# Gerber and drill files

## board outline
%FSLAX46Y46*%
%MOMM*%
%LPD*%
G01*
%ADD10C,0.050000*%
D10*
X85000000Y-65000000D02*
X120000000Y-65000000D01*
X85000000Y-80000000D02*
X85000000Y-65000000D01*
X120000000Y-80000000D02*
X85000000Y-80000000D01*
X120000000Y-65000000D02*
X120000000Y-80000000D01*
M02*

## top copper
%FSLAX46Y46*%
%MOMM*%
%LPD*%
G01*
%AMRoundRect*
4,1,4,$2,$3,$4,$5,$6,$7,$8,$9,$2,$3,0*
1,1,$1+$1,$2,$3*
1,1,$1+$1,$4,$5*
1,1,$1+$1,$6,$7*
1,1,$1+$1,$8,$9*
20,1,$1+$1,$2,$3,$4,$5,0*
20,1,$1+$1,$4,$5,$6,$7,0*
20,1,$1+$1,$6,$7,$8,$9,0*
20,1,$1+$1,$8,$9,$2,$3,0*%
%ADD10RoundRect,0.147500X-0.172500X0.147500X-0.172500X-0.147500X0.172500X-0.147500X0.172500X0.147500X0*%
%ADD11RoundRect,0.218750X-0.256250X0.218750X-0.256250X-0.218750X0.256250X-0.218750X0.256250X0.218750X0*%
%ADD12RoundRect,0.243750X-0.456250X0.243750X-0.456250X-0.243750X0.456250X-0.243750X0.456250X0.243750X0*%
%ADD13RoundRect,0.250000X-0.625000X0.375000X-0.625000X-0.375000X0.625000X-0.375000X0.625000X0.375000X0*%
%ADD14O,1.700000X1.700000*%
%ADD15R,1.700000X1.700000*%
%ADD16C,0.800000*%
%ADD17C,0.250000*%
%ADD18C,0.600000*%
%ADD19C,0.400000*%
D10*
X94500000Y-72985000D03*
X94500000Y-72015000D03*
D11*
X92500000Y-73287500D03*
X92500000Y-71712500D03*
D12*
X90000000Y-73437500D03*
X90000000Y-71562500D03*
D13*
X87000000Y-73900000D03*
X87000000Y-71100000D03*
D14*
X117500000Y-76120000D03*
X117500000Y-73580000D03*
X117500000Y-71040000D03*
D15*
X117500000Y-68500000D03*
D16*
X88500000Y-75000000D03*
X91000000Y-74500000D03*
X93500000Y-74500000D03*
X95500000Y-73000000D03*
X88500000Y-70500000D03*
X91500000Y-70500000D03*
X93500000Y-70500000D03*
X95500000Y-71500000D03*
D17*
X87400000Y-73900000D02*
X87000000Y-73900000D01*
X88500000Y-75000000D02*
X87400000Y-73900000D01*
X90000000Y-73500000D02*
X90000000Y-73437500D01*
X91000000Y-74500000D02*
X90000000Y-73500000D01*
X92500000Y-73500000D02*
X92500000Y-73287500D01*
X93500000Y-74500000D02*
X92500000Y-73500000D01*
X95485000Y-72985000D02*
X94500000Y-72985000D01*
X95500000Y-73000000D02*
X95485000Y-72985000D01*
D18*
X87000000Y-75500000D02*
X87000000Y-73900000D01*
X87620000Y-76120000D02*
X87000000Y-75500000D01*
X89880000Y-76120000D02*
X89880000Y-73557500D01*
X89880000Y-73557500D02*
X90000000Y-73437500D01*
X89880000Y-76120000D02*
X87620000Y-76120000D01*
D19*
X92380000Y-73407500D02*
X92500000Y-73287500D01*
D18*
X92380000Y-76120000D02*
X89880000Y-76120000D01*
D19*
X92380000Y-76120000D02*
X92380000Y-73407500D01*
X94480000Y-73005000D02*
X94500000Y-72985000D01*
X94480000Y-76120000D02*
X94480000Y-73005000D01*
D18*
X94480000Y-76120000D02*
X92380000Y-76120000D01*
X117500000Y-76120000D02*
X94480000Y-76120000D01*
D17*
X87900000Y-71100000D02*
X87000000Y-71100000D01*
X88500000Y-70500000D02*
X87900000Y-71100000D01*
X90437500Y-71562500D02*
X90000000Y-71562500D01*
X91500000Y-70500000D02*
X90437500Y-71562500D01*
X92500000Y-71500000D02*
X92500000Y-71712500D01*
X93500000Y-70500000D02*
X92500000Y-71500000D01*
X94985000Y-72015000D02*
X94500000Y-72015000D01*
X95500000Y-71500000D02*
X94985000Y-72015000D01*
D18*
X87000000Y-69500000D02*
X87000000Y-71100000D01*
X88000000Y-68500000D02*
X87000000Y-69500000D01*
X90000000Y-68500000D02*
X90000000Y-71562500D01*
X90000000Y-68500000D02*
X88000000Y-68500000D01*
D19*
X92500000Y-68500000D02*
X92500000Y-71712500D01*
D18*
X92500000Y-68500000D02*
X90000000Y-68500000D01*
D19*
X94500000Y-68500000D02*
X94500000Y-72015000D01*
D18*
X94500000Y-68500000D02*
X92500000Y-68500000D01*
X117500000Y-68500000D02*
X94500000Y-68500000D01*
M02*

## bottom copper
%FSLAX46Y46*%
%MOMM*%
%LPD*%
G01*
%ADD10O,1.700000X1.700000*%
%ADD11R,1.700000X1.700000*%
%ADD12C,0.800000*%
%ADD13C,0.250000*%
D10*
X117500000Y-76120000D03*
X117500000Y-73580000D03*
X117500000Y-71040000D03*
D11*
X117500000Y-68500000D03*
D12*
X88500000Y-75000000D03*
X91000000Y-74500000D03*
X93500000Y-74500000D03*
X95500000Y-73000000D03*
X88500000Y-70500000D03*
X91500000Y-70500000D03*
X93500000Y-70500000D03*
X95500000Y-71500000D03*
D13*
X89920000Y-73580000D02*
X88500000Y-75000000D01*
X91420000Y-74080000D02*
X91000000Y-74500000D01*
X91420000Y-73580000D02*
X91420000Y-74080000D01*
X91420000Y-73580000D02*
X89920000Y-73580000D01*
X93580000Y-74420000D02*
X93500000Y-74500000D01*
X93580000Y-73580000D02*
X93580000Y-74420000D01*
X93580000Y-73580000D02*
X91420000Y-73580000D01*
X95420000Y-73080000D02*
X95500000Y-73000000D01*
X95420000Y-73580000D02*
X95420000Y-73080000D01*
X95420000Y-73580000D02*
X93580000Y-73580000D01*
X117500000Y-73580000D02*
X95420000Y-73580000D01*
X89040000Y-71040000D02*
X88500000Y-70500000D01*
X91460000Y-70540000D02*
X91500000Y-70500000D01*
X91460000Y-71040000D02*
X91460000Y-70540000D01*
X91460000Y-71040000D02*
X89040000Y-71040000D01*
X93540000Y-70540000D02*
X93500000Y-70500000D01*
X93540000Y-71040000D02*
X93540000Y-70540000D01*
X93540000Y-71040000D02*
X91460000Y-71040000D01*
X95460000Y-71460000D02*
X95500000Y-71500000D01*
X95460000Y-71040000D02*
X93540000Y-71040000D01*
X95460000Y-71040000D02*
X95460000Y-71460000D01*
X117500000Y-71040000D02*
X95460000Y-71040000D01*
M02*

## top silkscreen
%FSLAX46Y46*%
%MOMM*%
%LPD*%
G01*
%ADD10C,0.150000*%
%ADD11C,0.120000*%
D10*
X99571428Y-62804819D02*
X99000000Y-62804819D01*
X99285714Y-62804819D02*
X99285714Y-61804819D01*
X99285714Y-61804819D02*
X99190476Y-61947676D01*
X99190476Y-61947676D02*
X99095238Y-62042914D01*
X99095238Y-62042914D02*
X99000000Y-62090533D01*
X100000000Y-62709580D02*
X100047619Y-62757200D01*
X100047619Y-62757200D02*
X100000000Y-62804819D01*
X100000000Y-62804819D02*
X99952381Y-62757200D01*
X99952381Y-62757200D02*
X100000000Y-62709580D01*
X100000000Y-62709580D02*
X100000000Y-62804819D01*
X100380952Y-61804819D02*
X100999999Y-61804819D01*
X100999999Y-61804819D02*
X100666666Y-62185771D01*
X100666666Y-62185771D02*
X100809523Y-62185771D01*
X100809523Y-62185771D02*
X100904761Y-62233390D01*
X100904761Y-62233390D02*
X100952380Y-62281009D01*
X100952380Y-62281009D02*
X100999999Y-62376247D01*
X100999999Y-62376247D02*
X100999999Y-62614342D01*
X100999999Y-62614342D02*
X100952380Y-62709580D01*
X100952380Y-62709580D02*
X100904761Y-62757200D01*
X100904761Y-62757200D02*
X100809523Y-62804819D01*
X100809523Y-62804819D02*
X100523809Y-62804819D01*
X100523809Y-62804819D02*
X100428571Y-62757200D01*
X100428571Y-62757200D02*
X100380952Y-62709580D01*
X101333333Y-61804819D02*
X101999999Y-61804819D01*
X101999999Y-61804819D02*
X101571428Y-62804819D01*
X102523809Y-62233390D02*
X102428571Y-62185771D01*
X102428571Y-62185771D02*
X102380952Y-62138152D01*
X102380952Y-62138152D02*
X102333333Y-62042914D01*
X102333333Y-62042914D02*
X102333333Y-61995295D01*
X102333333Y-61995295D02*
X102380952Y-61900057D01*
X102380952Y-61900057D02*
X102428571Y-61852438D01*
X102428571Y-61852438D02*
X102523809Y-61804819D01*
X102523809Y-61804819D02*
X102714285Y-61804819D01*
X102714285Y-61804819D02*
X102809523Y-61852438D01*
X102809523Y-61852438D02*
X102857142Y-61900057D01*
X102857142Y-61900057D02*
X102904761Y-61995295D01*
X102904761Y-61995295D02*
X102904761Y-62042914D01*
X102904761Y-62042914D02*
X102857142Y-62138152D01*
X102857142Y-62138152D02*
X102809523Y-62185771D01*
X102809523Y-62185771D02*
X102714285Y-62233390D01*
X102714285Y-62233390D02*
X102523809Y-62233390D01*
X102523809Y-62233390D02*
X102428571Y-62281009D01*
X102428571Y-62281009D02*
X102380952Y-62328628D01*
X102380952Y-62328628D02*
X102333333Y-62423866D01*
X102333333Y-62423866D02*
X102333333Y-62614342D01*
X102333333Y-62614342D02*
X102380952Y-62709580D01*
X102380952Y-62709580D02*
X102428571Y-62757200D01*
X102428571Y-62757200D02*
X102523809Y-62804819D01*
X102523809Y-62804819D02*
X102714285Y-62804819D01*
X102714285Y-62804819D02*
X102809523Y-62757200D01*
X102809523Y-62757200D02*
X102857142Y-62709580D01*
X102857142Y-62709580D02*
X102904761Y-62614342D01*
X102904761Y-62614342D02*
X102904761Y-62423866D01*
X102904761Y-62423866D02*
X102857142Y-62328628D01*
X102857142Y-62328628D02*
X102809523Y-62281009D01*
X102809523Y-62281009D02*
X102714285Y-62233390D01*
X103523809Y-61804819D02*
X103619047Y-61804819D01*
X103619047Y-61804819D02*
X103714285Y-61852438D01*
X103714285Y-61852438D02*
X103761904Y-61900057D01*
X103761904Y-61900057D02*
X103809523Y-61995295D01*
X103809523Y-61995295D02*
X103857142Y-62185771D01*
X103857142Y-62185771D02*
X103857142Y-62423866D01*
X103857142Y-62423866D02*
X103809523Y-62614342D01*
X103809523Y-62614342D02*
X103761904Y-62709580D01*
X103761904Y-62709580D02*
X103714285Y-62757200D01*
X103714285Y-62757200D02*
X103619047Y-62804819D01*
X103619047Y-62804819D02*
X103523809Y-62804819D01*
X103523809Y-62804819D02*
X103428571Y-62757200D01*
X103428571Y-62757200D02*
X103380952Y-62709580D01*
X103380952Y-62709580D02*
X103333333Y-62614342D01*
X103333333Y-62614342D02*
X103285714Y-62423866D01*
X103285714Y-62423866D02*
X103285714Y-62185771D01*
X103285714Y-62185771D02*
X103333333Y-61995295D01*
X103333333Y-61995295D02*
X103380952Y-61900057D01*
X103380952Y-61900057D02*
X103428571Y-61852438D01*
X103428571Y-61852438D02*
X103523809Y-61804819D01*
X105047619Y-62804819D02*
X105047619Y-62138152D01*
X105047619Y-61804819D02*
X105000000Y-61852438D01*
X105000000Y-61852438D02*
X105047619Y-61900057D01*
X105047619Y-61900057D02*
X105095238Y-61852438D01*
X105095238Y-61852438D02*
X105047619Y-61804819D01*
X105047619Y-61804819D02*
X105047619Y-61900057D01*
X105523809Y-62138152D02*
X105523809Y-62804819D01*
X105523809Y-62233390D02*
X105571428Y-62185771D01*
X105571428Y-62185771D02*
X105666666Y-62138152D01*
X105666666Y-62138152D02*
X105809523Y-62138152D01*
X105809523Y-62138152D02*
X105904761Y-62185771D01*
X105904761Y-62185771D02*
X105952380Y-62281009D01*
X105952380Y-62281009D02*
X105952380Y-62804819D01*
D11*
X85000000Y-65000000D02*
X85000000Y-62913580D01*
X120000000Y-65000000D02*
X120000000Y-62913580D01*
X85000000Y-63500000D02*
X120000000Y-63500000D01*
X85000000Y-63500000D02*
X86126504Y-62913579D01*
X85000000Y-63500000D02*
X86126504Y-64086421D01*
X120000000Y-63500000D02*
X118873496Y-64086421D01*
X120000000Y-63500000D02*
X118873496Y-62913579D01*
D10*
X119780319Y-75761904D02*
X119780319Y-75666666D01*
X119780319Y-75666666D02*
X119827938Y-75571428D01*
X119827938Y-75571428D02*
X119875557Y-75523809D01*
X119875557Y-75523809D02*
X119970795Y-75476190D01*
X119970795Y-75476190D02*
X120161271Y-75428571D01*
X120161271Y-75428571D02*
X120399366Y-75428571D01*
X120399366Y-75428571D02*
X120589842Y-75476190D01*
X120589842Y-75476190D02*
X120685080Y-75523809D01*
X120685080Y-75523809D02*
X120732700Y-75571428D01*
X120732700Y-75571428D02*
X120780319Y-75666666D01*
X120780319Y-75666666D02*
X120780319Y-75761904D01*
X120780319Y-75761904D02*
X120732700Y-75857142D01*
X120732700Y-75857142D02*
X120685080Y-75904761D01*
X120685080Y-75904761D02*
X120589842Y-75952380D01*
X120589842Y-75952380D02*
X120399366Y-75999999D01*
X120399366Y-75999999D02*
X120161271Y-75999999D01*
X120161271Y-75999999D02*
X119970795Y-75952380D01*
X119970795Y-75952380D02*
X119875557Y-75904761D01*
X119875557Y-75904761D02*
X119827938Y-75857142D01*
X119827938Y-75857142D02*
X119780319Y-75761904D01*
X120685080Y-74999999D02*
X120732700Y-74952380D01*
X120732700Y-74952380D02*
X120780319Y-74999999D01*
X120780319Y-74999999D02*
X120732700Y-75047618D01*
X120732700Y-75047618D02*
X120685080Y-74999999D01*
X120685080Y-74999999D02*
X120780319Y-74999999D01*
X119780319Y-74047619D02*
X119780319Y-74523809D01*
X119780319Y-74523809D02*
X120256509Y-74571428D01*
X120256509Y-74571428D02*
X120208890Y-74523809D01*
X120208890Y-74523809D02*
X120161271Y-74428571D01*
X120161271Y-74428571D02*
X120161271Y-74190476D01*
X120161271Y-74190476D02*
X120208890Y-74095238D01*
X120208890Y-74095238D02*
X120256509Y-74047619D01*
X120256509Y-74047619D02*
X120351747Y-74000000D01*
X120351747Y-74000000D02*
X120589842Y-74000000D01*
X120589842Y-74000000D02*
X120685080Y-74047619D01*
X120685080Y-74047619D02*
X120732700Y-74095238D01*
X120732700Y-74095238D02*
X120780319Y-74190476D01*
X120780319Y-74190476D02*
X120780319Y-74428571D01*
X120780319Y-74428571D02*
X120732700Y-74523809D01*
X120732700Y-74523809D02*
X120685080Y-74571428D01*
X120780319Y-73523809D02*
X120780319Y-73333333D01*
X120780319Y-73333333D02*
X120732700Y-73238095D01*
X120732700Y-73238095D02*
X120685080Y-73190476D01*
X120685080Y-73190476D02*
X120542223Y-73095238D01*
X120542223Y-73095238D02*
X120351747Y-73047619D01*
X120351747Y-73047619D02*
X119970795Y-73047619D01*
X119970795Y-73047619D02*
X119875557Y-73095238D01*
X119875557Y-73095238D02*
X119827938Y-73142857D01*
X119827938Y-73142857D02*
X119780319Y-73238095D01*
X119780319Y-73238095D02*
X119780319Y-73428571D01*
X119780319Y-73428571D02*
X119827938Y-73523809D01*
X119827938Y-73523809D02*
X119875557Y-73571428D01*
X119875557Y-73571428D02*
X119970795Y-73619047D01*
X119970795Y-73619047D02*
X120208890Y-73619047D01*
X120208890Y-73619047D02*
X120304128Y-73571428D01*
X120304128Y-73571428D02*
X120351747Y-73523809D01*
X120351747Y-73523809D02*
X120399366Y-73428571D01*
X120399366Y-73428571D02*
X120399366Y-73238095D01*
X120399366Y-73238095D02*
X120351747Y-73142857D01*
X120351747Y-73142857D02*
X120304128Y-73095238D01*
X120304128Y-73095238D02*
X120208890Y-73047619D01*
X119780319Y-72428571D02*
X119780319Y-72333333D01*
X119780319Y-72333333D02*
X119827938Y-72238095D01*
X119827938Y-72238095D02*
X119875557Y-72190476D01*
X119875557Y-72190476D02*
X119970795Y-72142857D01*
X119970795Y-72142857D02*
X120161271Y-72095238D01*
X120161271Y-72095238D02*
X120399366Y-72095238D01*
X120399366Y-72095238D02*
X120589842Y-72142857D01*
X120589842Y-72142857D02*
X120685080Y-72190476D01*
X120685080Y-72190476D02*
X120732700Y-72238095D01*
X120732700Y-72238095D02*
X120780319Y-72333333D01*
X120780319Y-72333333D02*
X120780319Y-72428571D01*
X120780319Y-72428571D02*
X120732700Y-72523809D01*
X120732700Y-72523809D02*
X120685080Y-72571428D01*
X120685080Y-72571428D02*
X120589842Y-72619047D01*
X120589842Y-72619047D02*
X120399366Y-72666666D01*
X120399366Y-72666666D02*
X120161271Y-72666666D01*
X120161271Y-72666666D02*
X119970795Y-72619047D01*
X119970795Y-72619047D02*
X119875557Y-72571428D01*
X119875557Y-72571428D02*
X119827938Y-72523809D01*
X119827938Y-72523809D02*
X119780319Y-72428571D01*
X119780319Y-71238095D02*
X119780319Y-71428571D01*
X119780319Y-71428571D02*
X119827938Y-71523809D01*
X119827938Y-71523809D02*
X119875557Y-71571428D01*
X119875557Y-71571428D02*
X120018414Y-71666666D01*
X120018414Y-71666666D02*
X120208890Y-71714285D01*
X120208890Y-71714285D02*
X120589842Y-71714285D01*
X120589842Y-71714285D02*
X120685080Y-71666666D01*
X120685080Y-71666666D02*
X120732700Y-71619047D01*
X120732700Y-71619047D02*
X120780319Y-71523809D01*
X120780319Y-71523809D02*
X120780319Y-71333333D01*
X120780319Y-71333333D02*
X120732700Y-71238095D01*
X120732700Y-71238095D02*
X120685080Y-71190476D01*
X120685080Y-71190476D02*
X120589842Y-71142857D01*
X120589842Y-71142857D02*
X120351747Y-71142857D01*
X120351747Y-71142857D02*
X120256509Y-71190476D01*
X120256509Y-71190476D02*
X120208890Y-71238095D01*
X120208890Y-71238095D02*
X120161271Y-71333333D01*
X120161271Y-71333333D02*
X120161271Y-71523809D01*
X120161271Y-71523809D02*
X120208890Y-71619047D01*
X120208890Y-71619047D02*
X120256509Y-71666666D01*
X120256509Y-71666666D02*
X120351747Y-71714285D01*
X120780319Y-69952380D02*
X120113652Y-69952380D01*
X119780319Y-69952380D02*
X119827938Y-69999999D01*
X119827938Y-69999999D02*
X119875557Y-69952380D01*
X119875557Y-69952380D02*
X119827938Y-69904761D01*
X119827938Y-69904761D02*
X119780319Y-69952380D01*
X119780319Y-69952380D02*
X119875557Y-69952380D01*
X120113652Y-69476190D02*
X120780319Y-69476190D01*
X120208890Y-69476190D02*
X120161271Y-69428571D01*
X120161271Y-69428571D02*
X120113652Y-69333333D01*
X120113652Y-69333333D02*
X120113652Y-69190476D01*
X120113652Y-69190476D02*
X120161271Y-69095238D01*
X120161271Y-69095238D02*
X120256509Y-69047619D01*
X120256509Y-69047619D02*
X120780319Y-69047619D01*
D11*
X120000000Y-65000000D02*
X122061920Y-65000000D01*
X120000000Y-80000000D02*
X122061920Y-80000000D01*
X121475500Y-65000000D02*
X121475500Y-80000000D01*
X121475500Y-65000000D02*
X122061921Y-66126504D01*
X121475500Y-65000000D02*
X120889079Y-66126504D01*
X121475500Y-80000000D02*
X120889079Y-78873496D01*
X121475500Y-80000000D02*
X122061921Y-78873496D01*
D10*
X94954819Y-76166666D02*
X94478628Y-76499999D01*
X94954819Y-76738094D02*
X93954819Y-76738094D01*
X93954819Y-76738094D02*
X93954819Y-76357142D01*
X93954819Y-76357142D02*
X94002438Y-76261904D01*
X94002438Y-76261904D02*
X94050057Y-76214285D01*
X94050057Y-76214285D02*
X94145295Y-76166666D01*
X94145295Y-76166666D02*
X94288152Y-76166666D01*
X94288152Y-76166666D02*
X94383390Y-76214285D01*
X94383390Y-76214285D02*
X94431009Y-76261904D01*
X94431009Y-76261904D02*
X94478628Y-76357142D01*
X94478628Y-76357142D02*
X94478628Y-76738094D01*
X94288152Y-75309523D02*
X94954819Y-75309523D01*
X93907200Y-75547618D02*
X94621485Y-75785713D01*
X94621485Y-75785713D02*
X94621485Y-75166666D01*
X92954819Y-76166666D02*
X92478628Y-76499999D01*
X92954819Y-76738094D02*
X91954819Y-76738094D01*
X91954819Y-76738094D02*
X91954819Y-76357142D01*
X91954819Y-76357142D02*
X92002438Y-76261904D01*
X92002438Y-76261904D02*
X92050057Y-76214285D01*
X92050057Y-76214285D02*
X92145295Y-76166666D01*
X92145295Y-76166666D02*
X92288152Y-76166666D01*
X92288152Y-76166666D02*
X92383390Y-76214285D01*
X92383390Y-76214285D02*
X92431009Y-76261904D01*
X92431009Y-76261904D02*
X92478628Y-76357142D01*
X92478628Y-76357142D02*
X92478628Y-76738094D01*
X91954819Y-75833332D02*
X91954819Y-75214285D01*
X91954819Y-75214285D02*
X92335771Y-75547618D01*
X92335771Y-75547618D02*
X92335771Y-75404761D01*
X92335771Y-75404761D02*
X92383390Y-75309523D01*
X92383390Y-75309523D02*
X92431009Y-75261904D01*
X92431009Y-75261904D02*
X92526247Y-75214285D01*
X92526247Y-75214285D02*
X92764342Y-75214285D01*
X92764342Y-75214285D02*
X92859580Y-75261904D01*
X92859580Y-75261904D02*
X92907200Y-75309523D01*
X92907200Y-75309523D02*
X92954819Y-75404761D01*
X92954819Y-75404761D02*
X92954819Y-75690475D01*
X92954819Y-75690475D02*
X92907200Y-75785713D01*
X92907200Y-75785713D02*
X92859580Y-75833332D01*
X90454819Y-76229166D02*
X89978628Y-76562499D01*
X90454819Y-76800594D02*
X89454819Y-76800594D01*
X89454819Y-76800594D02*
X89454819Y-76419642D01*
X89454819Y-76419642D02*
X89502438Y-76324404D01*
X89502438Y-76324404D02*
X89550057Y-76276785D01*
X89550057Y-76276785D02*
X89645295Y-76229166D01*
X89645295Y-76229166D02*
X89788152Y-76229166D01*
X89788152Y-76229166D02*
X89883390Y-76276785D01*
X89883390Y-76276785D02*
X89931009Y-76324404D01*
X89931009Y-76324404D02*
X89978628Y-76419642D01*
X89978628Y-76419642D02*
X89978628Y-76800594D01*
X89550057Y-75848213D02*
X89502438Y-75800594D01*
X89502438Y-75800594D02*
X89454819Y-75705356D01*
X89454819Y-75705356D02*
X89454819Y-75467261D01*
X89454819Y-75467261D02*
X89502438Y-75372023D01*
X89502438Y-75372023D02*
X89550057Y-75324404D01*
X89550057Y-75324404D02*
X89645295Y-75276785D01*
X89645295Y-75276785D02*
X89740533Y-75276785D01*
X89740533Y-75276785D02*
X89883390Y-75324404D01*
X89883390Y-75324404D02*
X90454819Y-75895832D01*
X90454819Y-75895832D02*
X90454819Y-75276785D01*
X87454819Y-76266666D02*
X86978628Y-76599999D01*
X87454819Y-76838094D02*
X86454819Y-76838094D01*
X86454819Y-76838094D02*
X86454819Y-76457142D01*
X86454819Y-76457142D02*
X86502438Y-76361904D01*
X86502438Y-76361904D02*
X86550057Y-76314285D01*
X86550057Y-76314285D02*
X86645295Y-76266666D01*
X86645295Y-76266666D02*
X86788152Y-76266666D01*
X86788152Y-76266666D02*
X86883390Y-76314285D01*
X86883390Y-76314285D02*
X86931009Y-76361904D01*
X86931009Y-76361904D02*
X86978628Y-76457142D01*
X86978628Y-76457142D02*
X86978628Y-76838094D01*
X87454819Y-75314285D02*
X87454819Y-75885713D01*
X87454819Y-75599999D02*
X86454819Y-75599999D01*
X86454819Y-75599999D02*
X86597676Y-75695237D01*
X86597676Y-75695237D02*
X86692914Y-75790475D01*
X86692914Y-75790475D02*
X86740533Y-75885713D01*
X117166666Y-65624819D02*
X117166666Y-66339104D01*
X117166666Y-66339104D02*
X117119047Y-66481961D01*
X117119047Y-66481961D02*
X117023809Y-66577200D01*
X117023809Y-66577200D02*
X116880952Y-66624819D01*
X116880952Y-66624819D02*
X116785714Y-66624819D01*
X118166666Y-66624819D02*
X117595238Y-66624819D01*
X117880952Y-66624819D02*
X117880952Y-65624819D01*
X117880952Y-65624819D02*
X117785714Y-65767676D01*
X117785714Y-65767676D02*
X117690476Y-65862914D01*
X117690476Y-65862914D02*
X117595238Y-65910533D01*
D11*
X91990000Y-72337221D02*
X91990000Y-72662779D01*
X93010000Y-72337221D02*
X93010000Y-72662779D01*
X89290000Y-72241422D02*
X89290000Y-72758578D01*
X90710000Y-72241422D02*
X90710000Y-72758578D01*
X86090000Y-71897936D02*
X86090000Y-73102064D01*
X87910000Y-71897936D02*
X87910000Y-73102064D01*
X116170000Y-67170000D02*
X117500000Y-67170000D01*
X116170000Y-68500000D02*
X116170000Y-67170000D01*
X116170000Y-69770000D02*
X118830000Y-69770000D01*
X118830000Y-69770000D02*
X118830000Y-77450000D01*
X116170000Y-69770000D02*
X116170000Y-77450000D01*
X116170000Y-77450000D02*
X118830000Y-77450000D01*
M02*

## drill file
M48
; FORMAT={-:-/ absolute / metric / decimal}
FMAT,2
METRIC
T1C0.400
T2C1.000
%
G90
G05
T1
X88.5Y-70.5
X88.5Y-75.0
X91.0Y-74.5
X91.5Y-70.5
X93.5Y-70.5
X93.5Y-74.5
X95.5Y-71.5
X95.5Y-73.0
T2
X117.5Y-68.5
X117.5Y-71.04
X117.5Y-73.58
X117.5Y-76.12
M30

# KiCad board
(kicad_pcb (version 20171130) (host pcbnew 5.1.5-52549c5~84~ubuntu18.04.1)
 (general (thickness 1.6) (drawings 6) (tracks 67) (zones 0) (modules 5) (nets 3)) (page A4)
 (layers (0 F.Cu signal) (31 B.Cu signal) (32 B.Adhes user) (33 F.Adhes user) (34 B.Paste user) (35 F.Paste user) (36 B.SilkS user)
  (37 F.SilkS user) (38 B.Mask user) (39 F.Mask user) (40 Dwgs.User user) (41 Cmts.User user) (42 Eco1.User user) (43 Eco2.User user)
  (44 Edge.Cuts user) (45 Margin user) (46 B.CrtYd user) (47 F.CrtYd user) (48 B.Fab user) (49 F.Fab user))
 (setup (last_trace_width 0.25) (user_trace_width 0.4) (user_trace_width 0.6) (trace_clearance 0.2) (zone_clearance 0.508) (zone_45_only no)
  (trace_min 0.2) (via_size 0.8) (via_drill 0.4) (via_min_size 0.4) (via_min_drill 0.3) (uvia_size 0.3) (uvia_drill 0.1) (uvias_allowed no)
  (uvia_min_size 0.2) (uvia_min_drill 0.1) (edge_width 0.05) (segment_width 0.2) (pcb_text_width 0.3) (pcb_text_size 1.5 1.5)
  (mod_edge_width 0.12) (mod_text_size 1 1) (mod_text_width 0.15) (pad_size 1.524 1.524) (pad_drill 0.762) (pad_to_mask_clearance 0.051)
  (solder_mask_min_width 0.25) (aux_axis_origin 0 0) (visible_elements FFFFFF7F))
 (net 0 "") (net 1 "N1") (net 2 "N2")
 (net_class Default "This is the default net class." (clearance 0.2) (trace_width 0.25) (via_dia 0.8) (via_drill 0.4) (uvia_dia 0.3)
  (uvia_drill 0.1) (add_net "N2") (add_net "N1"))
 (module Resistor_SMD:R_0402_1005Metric (layer F.Cu) (at 94.5 72.5 270)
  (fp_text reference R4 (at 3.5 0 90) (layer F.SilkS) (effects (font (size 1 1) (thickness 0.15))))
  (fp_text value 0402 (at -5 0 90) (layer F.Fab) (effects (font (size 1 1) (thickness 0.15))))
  (pad 2 smd roundrect (at 0.485 0 270) (size 0.59 0.64) (layers F.Cu F.Paste F.Mask) (roundrect_rratio 0.25) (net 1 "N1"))
  (pad 1 smd roundrect (at -0.485 0 270) (size 0.59 0.64) (layers F.Cu F.Paste F.Mask) (roundrect_rratio 0.25) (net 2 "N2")))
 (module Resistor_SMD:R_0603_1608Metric (layer F.Cu) (at 92.5 72.5 270)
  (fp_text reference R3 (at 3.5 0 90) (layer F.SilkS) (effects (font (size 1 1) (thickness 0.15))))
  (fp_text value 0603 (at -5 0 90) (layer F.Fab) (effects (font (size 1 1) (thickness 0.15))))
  (fp_line (start -0.162779 0.51) (end 0.162779 0.51) (layer F.SilkS) (width 0.12))
  (fp_line (start -0.162779 -0.51) (end 0.162779 -0.51) (layer F.SilkS) (width 0.12))
  (pad 2 smd roundrect (at 0.7875 0 270) (size 0.875 0.95) (layers F.Cu F.Paste F.Mask) (roundrect_rratio 0.25) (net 1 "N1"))
  (pad 1 smd roundrect (at -0.7875 0 270) (size 0.875 0.95) (layers F.Cu F.Paste F.Mask) (roundrect_rratio 0.25) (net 2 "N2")))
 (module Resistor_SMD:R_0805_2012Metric (layer F.Cu) (at 90 72.5 270)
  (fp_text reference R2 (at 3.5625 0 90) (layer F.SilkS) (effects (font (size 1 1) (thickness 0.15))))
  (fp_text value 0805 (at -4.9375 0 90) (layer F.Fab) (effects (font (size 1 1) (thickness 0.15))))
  (fp_line (start -0.258578 0.71) (end 0.258578 0.71) (layer F.SilkS) (width 0.12))
  (fp_line (start -0.258578 -0.71) (end 0.258578 -0.71) (layer F.SilkS) (width 0.12))
  (pad 2 smd roundrect (at 0.9375 0 270) (size 0.975 1.4) (layers F.Cu F.Paste F.Mask) (roundrect_rratio 0.25) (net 1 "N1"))
  (pad 1 smd roundrect (at -0.9375 0 270) (size 0.975 1.4) (layers F.Cu F.Paste F.Mask) (roundrect_rratio 0.25) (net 2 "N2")))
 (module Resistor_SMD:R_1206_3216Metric (layer F.Cu) (at 87 72.5 270)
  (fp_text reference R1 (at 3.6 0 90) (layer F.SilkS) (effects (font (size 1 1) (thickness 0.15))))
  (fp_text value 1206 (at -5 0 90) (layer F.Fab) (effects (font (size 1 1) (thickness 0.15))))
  (fp_line (start -0.602064 0.91) (end 0.602064 0.91) (layer F.SilkS) (width 0.12))
  (fp_line (start -0.602064 -0.91) (end 0.602064 -0.91) (layer F.SilkS) (width 0.12))
  (pad 2 smd roundrect (at 1.4 0 270) (size 1.25 1.75) (layers F.Cu F.Paste F.Mask) (roundrect_rratio 0.2) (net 1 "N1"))
  (pad 1 smd roundrect (at -1.4 0 270) (size 1.25 1.75) (layers F.Cu F.Paste F.Mask) (roundrect_rratio 0.2) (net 2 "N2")))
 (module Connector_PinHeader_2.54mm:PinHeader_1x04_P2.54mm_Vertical (layer F.Cu) (at 117.5 68.5)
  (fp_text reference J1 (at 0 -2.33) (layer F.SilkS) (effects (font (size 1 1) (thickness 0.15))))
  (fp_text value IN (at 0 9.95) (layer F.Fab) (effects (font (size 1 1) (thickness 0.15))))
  (fp_line (start -1.33 -1.33) (end 0 -1.33) (layer F.SilkS) (width 0.12))
  (fp_line (start -1.33 0) (end -1.33 -1.33) (layer F.SilkS) (width 0.12))
  (fp_line (start -1.33 1.27) (end 1.33 1.27) (layer F.SilkS) (width 0.12))
  (fp_line (start 1.33 1.27) (end 1.33 8.95) (layer F.SilkS) (width 0.12))
  (fp_line (start -1.33 1.27) (end -1.33 8.95) (layer F.SilkS) (width 0.12))
  (fp_line (start -1.33 8.95) (end 1.33 8.95) (layer F.SilkS) (width 0.12))
  (pad 4 thru_hole oval (at 0 7.62) (size 1.7 1.7) (drill 1) (layers *.Cu *.Mask) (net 1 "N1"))
  (pad 3 thru_hole oval (at 0 5.08) (size 1.7 1.7) (drill 1) (layers *.Cu *.Mask) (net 1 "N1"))
  (pad 2 thru_hole oval (at 0 2.54) (size 1.7 1.7) (drill 1) (layers *.Cu *.Mask) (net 2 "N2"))
  (pad 1 thru_hole rect (at 0 0) (size 1.7 1.7) (drill 1) (layers *.Cu *.Mask) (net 2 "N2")))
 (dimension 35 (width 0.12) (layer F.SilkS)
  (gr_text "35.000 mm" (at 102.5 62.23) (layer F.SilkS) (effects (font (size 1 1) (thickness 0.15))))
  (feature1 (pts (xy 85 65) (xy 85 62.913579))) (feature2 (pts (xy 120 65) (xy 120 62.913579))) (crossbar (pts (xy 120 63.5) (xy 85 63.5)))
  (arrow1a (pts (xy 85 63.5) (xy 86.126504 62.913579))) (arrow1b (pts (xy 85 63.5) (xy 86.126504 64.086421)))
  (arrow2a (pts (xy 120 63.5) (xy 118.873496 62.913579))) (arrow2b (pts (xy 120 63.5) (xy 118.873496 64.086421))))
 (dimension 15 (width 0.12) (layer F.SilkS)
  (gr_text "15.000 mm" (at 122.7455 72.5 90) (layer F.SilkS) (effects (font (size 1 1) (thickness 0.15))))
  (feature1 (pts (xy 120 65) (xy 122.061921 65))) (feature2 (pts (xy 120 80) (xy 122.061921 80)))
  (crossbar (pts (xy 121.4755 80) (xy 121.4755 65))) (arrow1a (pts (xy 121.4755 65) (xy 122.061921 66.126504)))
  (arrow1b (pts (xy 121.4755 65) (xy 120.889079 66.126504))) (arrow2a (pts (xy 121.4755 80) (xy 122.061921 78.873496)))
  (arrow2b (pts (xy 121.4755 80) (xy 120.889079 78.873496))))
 (gr_line (start 85 65) (end 120 65) (layer Edge.Cuts) (width 0.05))
 (gr_line (start 85 80) (end 85 65) (layer Edge.Cuts) (width 0.05))
 (gr_line (start 120 80) (end 85 80) (layer Edge.Cuts) (width 0.05))
 (gr_line (start 120 65) (end 120 80) (layer Edge.Cuts) (width 0.05))
 (via (at 88.5 75) (size 0.8) (drill 0.4) (layers F.Cu B.Cu) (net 1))
 (segment (start 89.92 73.58) (end 88.5 75) (width 0.25) (layer B.Cu) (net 1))
 (segment (start 87.4 73.9) (end 87 73.9) (width 0.25) (layer F.Cu) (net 1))
 (segment (start 88.5 75) (end 87.4 73.9) (width 0.25) (layer F.Cu) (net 1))
 (via (at 91 74.5) (size 0.8) (drill 0.4) (layers F.Cu B.Cu) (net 1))
 (segment (start 91.42 74.08) (end 91 74.5) (width 0.25) (layer B.Cu) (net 1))
 (segment (start 91.42 73.58) (end 91.42 74.08) (width 0.25) (layer B.Cu) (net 1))
 (segment (start 91.42 73.58) (end 89.92 73.58) (width 0.25) (layer B.Cu) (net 1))
 (segment (start 90 73.5) (end 90 73.4375) (width 0.25) (layer F.Cu) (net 1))
 (segment (start 91 74.5) (end 90 73.5) (width 0.25) (layer F.Cu) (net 1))
 (via (at 93.5 74.5) (size 0.8) (drill 0.4) (layers F.Cu B.Cu) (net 1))
 (segment (start 93.58 74.42) (end 93.5 74.5) (width 0.25) (layer B.Cu) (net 1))
 (segment (start 93.58 73.58) (end 93.58 74.42) (width 0.25) (layer B.Cu) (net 1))
 (segment (start 93.58 73.58) (end 91.42 73.58) (width 0.25) (layer B.Cu) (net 1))
 (segment (start 92.5 73.5) (end 92.5 73.2875) (width 0.25) (layer F.Cu) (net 1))
 (segment (start 93.5 74.5) (end 92.5 73.5) (width 0.25) (layer F.Cu) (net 1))
 (via (at 95.5 73) (size 0.8) (drill 0.4) (layers F.Cu B.Cu) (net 1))
 (segment (start 95.42 73.08) (end 95.5 73) (width 0.25) (layer B.Cu) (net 1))
 (segment (start 95.42 73.58) (end 95.42 73.08) (width 0.25) (layer B.Cu) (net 1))
 (segment (start 95.42 73.58) (end 93.58 73.58) (width 0.25) (layer B.Cu) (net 1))
 (segment (start 117.5 73.58) (end 95.42 73.58) (width 0.25) (layer B.Cu) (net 1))
 (segment (start 95.485 72.985) (end 94.5 72.985) (width 0.25) (layer F.Cu) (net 1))
 (segment (start 95.5 73) (end 95.485 72.985) (width 0.25) (layer F.Cu) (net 1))
 (segment (start 87 75.5) (end 87 73.9) (width 0.6) (layer F.Cu) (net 1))
 (segment (start 87.62 76.12) (end 87 75.5) (width 0.6) (layer F.Cu) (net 1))
 (segment (start 89.88 76.12) (end 89.88 73.5575) (width 0.6) (layer F.Cu) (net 1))
 (segment (start 89.88 73.5575) (end 90 73.4375) (width 0.6) (layer F.Cu) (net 1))
 (segment (start 89.88 76.12) (end 87.62 76.12) (width 0.6) (layer F.Cu) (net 1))
 (segment (start 92.38 73.4075) (end 92.5 73.2875) (width 0.4) (layer F.Cu) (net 1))
 (segment (start 92.38 76.12) (end 89.88 76.12) (width 0.6) (layer F.Cu) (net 1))
 (segment (start 92.38 76.12) (end 92.38 73.4075) (width 0.4) (layer F.Cu) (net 1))
 (segment (start 94.48 73.005) (end 94.5 72.985) (width 0.4) (layer F.Cu) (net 1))
 (segment (start 94.48 76.12) (end 94.48 73.005) (width 0.4) (layer F.Cu) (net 1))
 (segment (start 94.48 76.12) (end 92.38 76.12) (width 0.6) (layer F.Cu) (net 1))
 (segment (start 117.5 76.12) (end 94.48 76.12) (width 0.6) (layer F.Cu) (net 1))
 (via (at 88.5 70.5) (size 0.8) (drill 0.4) (layers F.Cu B.Cu) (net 2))
 (segment (start 89.04 71.04) (end 88.5 70.5) (width 0.25) (layer B.Cu) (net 2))
 (segment (start 87.9 71.1) (end 87 71.1) (width 0.25) (layer F.Cu) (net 2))
 (segment (start 88.5 70.5) (end 87.9 71.1) (width 0.25) (layer F.Cu) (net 2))
 (segment (start 91.46 70.54) (end 91.5 70.5) (width 0.25) (layer B.Cu) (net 2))
 (via (at 91.5 70.5) (size 0.8) (drill 0.4) (layers F.Cu B.Cu) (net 2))
 (segment (start 91.46 71.04) (end 91.46 70.54) (width 0.25) (layer B.Cu) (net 2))
 (segment (start 91.46 71.04) (end 89.04 71.04) (width 0.25) (layer B.Cu) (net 2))
 (segment (start 90.4375 71.5625) (end 90 71.5625) (width 0.25) (layer F.Cu) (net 2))
 (segment (start 91.5 70.5) (end 90.4375 71.5625) (width 0.25) (layer F.Cu) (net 2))
 (segment (start 93.54 70.54) (end 93.5 70.5) (width 0.25) (layer B.Cu) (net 2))
 (segment (start 93.54 71.04) (end 93.54 70.54) (width 0.25) (layer B.Cu) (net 2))
 (via (at 93.5 70.5) (size 0.8) (drill 0.4) (layers F.Cu B.Cu) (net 2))
 (segment (start 93.54 71.04) (end 91.46 71.04) (width 0.25) (layer B.Cu) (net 2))
 (segment (start 92.5 71.5) (end 92.5 71.7125) (width 0.25) (layer F.Cu) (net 2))
 (segment (start 93.5 70.5) (end 92.5 71.5) (width 0.25) (layer F.Cu) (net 2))
 (via (at 95.5 71.5) (size 0.8) (drill 0.4) (layers F.Cu B.Cu) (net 2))
 (segment (start 95.46 71.46) (end 95.5 71.5) (width 0.25) (layer B.Cu) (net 2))
 (segment (start 95.46 71.04) (end 93.54 71.04) (width 0.25) (layer B.Cu) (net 2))
 (segment (start 95.46 71.04) (end 95.46 71.46) (width 0.25) (layer B.Cu) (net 2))
 (segment (start 117.5 71.04) (end 95.46 71.04) (width 0.25) (layer B.Cu) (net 2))
 (segment (start 94.985 72.015) (end 94.5 72.015) (width 0.25) (layer F.Cu) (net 2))
 (segment (start 95.5 71.5) (end 94.985 72.015) (width 0.25) (layer F.Cu) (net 2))
 (segment (start 87 69.5) (end 87 71.1) (width 0.6) (layer F.Cu) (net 2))
 (segment (start 88 68.5) (end 87 69.5) (width 0.6) (layer F.Cu) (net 2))
 (segment (start 90 68.5) (end 90 71.5625) (width 0.6) (layer F.Cu) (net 2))
 (segment (start 90 68.5) (end 88 68.5) (width 0.6) (layer F.Cu) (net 2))
 (segment (start 92.5 68.5) (end 92.5 71.7125) (width 0.4) (layer F.Cu) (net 2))
 (segment (start 92.5 68.5) (end 90 68.5) (width 0.6) (layer F.Cu) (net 2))
 (segment (start 94.5 68.5) (end 94.5 72.015) (width 0.4) (layer F.Cu) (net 2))
 (segment (start 94.5 68.5) (end 92.5 68.5) (width 0.6) (layer F.Cu) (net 2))
 (segment (start 117.5 68.5) (end 94.5 68.5) (width 0.6) (layer F.Cu) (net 2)))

